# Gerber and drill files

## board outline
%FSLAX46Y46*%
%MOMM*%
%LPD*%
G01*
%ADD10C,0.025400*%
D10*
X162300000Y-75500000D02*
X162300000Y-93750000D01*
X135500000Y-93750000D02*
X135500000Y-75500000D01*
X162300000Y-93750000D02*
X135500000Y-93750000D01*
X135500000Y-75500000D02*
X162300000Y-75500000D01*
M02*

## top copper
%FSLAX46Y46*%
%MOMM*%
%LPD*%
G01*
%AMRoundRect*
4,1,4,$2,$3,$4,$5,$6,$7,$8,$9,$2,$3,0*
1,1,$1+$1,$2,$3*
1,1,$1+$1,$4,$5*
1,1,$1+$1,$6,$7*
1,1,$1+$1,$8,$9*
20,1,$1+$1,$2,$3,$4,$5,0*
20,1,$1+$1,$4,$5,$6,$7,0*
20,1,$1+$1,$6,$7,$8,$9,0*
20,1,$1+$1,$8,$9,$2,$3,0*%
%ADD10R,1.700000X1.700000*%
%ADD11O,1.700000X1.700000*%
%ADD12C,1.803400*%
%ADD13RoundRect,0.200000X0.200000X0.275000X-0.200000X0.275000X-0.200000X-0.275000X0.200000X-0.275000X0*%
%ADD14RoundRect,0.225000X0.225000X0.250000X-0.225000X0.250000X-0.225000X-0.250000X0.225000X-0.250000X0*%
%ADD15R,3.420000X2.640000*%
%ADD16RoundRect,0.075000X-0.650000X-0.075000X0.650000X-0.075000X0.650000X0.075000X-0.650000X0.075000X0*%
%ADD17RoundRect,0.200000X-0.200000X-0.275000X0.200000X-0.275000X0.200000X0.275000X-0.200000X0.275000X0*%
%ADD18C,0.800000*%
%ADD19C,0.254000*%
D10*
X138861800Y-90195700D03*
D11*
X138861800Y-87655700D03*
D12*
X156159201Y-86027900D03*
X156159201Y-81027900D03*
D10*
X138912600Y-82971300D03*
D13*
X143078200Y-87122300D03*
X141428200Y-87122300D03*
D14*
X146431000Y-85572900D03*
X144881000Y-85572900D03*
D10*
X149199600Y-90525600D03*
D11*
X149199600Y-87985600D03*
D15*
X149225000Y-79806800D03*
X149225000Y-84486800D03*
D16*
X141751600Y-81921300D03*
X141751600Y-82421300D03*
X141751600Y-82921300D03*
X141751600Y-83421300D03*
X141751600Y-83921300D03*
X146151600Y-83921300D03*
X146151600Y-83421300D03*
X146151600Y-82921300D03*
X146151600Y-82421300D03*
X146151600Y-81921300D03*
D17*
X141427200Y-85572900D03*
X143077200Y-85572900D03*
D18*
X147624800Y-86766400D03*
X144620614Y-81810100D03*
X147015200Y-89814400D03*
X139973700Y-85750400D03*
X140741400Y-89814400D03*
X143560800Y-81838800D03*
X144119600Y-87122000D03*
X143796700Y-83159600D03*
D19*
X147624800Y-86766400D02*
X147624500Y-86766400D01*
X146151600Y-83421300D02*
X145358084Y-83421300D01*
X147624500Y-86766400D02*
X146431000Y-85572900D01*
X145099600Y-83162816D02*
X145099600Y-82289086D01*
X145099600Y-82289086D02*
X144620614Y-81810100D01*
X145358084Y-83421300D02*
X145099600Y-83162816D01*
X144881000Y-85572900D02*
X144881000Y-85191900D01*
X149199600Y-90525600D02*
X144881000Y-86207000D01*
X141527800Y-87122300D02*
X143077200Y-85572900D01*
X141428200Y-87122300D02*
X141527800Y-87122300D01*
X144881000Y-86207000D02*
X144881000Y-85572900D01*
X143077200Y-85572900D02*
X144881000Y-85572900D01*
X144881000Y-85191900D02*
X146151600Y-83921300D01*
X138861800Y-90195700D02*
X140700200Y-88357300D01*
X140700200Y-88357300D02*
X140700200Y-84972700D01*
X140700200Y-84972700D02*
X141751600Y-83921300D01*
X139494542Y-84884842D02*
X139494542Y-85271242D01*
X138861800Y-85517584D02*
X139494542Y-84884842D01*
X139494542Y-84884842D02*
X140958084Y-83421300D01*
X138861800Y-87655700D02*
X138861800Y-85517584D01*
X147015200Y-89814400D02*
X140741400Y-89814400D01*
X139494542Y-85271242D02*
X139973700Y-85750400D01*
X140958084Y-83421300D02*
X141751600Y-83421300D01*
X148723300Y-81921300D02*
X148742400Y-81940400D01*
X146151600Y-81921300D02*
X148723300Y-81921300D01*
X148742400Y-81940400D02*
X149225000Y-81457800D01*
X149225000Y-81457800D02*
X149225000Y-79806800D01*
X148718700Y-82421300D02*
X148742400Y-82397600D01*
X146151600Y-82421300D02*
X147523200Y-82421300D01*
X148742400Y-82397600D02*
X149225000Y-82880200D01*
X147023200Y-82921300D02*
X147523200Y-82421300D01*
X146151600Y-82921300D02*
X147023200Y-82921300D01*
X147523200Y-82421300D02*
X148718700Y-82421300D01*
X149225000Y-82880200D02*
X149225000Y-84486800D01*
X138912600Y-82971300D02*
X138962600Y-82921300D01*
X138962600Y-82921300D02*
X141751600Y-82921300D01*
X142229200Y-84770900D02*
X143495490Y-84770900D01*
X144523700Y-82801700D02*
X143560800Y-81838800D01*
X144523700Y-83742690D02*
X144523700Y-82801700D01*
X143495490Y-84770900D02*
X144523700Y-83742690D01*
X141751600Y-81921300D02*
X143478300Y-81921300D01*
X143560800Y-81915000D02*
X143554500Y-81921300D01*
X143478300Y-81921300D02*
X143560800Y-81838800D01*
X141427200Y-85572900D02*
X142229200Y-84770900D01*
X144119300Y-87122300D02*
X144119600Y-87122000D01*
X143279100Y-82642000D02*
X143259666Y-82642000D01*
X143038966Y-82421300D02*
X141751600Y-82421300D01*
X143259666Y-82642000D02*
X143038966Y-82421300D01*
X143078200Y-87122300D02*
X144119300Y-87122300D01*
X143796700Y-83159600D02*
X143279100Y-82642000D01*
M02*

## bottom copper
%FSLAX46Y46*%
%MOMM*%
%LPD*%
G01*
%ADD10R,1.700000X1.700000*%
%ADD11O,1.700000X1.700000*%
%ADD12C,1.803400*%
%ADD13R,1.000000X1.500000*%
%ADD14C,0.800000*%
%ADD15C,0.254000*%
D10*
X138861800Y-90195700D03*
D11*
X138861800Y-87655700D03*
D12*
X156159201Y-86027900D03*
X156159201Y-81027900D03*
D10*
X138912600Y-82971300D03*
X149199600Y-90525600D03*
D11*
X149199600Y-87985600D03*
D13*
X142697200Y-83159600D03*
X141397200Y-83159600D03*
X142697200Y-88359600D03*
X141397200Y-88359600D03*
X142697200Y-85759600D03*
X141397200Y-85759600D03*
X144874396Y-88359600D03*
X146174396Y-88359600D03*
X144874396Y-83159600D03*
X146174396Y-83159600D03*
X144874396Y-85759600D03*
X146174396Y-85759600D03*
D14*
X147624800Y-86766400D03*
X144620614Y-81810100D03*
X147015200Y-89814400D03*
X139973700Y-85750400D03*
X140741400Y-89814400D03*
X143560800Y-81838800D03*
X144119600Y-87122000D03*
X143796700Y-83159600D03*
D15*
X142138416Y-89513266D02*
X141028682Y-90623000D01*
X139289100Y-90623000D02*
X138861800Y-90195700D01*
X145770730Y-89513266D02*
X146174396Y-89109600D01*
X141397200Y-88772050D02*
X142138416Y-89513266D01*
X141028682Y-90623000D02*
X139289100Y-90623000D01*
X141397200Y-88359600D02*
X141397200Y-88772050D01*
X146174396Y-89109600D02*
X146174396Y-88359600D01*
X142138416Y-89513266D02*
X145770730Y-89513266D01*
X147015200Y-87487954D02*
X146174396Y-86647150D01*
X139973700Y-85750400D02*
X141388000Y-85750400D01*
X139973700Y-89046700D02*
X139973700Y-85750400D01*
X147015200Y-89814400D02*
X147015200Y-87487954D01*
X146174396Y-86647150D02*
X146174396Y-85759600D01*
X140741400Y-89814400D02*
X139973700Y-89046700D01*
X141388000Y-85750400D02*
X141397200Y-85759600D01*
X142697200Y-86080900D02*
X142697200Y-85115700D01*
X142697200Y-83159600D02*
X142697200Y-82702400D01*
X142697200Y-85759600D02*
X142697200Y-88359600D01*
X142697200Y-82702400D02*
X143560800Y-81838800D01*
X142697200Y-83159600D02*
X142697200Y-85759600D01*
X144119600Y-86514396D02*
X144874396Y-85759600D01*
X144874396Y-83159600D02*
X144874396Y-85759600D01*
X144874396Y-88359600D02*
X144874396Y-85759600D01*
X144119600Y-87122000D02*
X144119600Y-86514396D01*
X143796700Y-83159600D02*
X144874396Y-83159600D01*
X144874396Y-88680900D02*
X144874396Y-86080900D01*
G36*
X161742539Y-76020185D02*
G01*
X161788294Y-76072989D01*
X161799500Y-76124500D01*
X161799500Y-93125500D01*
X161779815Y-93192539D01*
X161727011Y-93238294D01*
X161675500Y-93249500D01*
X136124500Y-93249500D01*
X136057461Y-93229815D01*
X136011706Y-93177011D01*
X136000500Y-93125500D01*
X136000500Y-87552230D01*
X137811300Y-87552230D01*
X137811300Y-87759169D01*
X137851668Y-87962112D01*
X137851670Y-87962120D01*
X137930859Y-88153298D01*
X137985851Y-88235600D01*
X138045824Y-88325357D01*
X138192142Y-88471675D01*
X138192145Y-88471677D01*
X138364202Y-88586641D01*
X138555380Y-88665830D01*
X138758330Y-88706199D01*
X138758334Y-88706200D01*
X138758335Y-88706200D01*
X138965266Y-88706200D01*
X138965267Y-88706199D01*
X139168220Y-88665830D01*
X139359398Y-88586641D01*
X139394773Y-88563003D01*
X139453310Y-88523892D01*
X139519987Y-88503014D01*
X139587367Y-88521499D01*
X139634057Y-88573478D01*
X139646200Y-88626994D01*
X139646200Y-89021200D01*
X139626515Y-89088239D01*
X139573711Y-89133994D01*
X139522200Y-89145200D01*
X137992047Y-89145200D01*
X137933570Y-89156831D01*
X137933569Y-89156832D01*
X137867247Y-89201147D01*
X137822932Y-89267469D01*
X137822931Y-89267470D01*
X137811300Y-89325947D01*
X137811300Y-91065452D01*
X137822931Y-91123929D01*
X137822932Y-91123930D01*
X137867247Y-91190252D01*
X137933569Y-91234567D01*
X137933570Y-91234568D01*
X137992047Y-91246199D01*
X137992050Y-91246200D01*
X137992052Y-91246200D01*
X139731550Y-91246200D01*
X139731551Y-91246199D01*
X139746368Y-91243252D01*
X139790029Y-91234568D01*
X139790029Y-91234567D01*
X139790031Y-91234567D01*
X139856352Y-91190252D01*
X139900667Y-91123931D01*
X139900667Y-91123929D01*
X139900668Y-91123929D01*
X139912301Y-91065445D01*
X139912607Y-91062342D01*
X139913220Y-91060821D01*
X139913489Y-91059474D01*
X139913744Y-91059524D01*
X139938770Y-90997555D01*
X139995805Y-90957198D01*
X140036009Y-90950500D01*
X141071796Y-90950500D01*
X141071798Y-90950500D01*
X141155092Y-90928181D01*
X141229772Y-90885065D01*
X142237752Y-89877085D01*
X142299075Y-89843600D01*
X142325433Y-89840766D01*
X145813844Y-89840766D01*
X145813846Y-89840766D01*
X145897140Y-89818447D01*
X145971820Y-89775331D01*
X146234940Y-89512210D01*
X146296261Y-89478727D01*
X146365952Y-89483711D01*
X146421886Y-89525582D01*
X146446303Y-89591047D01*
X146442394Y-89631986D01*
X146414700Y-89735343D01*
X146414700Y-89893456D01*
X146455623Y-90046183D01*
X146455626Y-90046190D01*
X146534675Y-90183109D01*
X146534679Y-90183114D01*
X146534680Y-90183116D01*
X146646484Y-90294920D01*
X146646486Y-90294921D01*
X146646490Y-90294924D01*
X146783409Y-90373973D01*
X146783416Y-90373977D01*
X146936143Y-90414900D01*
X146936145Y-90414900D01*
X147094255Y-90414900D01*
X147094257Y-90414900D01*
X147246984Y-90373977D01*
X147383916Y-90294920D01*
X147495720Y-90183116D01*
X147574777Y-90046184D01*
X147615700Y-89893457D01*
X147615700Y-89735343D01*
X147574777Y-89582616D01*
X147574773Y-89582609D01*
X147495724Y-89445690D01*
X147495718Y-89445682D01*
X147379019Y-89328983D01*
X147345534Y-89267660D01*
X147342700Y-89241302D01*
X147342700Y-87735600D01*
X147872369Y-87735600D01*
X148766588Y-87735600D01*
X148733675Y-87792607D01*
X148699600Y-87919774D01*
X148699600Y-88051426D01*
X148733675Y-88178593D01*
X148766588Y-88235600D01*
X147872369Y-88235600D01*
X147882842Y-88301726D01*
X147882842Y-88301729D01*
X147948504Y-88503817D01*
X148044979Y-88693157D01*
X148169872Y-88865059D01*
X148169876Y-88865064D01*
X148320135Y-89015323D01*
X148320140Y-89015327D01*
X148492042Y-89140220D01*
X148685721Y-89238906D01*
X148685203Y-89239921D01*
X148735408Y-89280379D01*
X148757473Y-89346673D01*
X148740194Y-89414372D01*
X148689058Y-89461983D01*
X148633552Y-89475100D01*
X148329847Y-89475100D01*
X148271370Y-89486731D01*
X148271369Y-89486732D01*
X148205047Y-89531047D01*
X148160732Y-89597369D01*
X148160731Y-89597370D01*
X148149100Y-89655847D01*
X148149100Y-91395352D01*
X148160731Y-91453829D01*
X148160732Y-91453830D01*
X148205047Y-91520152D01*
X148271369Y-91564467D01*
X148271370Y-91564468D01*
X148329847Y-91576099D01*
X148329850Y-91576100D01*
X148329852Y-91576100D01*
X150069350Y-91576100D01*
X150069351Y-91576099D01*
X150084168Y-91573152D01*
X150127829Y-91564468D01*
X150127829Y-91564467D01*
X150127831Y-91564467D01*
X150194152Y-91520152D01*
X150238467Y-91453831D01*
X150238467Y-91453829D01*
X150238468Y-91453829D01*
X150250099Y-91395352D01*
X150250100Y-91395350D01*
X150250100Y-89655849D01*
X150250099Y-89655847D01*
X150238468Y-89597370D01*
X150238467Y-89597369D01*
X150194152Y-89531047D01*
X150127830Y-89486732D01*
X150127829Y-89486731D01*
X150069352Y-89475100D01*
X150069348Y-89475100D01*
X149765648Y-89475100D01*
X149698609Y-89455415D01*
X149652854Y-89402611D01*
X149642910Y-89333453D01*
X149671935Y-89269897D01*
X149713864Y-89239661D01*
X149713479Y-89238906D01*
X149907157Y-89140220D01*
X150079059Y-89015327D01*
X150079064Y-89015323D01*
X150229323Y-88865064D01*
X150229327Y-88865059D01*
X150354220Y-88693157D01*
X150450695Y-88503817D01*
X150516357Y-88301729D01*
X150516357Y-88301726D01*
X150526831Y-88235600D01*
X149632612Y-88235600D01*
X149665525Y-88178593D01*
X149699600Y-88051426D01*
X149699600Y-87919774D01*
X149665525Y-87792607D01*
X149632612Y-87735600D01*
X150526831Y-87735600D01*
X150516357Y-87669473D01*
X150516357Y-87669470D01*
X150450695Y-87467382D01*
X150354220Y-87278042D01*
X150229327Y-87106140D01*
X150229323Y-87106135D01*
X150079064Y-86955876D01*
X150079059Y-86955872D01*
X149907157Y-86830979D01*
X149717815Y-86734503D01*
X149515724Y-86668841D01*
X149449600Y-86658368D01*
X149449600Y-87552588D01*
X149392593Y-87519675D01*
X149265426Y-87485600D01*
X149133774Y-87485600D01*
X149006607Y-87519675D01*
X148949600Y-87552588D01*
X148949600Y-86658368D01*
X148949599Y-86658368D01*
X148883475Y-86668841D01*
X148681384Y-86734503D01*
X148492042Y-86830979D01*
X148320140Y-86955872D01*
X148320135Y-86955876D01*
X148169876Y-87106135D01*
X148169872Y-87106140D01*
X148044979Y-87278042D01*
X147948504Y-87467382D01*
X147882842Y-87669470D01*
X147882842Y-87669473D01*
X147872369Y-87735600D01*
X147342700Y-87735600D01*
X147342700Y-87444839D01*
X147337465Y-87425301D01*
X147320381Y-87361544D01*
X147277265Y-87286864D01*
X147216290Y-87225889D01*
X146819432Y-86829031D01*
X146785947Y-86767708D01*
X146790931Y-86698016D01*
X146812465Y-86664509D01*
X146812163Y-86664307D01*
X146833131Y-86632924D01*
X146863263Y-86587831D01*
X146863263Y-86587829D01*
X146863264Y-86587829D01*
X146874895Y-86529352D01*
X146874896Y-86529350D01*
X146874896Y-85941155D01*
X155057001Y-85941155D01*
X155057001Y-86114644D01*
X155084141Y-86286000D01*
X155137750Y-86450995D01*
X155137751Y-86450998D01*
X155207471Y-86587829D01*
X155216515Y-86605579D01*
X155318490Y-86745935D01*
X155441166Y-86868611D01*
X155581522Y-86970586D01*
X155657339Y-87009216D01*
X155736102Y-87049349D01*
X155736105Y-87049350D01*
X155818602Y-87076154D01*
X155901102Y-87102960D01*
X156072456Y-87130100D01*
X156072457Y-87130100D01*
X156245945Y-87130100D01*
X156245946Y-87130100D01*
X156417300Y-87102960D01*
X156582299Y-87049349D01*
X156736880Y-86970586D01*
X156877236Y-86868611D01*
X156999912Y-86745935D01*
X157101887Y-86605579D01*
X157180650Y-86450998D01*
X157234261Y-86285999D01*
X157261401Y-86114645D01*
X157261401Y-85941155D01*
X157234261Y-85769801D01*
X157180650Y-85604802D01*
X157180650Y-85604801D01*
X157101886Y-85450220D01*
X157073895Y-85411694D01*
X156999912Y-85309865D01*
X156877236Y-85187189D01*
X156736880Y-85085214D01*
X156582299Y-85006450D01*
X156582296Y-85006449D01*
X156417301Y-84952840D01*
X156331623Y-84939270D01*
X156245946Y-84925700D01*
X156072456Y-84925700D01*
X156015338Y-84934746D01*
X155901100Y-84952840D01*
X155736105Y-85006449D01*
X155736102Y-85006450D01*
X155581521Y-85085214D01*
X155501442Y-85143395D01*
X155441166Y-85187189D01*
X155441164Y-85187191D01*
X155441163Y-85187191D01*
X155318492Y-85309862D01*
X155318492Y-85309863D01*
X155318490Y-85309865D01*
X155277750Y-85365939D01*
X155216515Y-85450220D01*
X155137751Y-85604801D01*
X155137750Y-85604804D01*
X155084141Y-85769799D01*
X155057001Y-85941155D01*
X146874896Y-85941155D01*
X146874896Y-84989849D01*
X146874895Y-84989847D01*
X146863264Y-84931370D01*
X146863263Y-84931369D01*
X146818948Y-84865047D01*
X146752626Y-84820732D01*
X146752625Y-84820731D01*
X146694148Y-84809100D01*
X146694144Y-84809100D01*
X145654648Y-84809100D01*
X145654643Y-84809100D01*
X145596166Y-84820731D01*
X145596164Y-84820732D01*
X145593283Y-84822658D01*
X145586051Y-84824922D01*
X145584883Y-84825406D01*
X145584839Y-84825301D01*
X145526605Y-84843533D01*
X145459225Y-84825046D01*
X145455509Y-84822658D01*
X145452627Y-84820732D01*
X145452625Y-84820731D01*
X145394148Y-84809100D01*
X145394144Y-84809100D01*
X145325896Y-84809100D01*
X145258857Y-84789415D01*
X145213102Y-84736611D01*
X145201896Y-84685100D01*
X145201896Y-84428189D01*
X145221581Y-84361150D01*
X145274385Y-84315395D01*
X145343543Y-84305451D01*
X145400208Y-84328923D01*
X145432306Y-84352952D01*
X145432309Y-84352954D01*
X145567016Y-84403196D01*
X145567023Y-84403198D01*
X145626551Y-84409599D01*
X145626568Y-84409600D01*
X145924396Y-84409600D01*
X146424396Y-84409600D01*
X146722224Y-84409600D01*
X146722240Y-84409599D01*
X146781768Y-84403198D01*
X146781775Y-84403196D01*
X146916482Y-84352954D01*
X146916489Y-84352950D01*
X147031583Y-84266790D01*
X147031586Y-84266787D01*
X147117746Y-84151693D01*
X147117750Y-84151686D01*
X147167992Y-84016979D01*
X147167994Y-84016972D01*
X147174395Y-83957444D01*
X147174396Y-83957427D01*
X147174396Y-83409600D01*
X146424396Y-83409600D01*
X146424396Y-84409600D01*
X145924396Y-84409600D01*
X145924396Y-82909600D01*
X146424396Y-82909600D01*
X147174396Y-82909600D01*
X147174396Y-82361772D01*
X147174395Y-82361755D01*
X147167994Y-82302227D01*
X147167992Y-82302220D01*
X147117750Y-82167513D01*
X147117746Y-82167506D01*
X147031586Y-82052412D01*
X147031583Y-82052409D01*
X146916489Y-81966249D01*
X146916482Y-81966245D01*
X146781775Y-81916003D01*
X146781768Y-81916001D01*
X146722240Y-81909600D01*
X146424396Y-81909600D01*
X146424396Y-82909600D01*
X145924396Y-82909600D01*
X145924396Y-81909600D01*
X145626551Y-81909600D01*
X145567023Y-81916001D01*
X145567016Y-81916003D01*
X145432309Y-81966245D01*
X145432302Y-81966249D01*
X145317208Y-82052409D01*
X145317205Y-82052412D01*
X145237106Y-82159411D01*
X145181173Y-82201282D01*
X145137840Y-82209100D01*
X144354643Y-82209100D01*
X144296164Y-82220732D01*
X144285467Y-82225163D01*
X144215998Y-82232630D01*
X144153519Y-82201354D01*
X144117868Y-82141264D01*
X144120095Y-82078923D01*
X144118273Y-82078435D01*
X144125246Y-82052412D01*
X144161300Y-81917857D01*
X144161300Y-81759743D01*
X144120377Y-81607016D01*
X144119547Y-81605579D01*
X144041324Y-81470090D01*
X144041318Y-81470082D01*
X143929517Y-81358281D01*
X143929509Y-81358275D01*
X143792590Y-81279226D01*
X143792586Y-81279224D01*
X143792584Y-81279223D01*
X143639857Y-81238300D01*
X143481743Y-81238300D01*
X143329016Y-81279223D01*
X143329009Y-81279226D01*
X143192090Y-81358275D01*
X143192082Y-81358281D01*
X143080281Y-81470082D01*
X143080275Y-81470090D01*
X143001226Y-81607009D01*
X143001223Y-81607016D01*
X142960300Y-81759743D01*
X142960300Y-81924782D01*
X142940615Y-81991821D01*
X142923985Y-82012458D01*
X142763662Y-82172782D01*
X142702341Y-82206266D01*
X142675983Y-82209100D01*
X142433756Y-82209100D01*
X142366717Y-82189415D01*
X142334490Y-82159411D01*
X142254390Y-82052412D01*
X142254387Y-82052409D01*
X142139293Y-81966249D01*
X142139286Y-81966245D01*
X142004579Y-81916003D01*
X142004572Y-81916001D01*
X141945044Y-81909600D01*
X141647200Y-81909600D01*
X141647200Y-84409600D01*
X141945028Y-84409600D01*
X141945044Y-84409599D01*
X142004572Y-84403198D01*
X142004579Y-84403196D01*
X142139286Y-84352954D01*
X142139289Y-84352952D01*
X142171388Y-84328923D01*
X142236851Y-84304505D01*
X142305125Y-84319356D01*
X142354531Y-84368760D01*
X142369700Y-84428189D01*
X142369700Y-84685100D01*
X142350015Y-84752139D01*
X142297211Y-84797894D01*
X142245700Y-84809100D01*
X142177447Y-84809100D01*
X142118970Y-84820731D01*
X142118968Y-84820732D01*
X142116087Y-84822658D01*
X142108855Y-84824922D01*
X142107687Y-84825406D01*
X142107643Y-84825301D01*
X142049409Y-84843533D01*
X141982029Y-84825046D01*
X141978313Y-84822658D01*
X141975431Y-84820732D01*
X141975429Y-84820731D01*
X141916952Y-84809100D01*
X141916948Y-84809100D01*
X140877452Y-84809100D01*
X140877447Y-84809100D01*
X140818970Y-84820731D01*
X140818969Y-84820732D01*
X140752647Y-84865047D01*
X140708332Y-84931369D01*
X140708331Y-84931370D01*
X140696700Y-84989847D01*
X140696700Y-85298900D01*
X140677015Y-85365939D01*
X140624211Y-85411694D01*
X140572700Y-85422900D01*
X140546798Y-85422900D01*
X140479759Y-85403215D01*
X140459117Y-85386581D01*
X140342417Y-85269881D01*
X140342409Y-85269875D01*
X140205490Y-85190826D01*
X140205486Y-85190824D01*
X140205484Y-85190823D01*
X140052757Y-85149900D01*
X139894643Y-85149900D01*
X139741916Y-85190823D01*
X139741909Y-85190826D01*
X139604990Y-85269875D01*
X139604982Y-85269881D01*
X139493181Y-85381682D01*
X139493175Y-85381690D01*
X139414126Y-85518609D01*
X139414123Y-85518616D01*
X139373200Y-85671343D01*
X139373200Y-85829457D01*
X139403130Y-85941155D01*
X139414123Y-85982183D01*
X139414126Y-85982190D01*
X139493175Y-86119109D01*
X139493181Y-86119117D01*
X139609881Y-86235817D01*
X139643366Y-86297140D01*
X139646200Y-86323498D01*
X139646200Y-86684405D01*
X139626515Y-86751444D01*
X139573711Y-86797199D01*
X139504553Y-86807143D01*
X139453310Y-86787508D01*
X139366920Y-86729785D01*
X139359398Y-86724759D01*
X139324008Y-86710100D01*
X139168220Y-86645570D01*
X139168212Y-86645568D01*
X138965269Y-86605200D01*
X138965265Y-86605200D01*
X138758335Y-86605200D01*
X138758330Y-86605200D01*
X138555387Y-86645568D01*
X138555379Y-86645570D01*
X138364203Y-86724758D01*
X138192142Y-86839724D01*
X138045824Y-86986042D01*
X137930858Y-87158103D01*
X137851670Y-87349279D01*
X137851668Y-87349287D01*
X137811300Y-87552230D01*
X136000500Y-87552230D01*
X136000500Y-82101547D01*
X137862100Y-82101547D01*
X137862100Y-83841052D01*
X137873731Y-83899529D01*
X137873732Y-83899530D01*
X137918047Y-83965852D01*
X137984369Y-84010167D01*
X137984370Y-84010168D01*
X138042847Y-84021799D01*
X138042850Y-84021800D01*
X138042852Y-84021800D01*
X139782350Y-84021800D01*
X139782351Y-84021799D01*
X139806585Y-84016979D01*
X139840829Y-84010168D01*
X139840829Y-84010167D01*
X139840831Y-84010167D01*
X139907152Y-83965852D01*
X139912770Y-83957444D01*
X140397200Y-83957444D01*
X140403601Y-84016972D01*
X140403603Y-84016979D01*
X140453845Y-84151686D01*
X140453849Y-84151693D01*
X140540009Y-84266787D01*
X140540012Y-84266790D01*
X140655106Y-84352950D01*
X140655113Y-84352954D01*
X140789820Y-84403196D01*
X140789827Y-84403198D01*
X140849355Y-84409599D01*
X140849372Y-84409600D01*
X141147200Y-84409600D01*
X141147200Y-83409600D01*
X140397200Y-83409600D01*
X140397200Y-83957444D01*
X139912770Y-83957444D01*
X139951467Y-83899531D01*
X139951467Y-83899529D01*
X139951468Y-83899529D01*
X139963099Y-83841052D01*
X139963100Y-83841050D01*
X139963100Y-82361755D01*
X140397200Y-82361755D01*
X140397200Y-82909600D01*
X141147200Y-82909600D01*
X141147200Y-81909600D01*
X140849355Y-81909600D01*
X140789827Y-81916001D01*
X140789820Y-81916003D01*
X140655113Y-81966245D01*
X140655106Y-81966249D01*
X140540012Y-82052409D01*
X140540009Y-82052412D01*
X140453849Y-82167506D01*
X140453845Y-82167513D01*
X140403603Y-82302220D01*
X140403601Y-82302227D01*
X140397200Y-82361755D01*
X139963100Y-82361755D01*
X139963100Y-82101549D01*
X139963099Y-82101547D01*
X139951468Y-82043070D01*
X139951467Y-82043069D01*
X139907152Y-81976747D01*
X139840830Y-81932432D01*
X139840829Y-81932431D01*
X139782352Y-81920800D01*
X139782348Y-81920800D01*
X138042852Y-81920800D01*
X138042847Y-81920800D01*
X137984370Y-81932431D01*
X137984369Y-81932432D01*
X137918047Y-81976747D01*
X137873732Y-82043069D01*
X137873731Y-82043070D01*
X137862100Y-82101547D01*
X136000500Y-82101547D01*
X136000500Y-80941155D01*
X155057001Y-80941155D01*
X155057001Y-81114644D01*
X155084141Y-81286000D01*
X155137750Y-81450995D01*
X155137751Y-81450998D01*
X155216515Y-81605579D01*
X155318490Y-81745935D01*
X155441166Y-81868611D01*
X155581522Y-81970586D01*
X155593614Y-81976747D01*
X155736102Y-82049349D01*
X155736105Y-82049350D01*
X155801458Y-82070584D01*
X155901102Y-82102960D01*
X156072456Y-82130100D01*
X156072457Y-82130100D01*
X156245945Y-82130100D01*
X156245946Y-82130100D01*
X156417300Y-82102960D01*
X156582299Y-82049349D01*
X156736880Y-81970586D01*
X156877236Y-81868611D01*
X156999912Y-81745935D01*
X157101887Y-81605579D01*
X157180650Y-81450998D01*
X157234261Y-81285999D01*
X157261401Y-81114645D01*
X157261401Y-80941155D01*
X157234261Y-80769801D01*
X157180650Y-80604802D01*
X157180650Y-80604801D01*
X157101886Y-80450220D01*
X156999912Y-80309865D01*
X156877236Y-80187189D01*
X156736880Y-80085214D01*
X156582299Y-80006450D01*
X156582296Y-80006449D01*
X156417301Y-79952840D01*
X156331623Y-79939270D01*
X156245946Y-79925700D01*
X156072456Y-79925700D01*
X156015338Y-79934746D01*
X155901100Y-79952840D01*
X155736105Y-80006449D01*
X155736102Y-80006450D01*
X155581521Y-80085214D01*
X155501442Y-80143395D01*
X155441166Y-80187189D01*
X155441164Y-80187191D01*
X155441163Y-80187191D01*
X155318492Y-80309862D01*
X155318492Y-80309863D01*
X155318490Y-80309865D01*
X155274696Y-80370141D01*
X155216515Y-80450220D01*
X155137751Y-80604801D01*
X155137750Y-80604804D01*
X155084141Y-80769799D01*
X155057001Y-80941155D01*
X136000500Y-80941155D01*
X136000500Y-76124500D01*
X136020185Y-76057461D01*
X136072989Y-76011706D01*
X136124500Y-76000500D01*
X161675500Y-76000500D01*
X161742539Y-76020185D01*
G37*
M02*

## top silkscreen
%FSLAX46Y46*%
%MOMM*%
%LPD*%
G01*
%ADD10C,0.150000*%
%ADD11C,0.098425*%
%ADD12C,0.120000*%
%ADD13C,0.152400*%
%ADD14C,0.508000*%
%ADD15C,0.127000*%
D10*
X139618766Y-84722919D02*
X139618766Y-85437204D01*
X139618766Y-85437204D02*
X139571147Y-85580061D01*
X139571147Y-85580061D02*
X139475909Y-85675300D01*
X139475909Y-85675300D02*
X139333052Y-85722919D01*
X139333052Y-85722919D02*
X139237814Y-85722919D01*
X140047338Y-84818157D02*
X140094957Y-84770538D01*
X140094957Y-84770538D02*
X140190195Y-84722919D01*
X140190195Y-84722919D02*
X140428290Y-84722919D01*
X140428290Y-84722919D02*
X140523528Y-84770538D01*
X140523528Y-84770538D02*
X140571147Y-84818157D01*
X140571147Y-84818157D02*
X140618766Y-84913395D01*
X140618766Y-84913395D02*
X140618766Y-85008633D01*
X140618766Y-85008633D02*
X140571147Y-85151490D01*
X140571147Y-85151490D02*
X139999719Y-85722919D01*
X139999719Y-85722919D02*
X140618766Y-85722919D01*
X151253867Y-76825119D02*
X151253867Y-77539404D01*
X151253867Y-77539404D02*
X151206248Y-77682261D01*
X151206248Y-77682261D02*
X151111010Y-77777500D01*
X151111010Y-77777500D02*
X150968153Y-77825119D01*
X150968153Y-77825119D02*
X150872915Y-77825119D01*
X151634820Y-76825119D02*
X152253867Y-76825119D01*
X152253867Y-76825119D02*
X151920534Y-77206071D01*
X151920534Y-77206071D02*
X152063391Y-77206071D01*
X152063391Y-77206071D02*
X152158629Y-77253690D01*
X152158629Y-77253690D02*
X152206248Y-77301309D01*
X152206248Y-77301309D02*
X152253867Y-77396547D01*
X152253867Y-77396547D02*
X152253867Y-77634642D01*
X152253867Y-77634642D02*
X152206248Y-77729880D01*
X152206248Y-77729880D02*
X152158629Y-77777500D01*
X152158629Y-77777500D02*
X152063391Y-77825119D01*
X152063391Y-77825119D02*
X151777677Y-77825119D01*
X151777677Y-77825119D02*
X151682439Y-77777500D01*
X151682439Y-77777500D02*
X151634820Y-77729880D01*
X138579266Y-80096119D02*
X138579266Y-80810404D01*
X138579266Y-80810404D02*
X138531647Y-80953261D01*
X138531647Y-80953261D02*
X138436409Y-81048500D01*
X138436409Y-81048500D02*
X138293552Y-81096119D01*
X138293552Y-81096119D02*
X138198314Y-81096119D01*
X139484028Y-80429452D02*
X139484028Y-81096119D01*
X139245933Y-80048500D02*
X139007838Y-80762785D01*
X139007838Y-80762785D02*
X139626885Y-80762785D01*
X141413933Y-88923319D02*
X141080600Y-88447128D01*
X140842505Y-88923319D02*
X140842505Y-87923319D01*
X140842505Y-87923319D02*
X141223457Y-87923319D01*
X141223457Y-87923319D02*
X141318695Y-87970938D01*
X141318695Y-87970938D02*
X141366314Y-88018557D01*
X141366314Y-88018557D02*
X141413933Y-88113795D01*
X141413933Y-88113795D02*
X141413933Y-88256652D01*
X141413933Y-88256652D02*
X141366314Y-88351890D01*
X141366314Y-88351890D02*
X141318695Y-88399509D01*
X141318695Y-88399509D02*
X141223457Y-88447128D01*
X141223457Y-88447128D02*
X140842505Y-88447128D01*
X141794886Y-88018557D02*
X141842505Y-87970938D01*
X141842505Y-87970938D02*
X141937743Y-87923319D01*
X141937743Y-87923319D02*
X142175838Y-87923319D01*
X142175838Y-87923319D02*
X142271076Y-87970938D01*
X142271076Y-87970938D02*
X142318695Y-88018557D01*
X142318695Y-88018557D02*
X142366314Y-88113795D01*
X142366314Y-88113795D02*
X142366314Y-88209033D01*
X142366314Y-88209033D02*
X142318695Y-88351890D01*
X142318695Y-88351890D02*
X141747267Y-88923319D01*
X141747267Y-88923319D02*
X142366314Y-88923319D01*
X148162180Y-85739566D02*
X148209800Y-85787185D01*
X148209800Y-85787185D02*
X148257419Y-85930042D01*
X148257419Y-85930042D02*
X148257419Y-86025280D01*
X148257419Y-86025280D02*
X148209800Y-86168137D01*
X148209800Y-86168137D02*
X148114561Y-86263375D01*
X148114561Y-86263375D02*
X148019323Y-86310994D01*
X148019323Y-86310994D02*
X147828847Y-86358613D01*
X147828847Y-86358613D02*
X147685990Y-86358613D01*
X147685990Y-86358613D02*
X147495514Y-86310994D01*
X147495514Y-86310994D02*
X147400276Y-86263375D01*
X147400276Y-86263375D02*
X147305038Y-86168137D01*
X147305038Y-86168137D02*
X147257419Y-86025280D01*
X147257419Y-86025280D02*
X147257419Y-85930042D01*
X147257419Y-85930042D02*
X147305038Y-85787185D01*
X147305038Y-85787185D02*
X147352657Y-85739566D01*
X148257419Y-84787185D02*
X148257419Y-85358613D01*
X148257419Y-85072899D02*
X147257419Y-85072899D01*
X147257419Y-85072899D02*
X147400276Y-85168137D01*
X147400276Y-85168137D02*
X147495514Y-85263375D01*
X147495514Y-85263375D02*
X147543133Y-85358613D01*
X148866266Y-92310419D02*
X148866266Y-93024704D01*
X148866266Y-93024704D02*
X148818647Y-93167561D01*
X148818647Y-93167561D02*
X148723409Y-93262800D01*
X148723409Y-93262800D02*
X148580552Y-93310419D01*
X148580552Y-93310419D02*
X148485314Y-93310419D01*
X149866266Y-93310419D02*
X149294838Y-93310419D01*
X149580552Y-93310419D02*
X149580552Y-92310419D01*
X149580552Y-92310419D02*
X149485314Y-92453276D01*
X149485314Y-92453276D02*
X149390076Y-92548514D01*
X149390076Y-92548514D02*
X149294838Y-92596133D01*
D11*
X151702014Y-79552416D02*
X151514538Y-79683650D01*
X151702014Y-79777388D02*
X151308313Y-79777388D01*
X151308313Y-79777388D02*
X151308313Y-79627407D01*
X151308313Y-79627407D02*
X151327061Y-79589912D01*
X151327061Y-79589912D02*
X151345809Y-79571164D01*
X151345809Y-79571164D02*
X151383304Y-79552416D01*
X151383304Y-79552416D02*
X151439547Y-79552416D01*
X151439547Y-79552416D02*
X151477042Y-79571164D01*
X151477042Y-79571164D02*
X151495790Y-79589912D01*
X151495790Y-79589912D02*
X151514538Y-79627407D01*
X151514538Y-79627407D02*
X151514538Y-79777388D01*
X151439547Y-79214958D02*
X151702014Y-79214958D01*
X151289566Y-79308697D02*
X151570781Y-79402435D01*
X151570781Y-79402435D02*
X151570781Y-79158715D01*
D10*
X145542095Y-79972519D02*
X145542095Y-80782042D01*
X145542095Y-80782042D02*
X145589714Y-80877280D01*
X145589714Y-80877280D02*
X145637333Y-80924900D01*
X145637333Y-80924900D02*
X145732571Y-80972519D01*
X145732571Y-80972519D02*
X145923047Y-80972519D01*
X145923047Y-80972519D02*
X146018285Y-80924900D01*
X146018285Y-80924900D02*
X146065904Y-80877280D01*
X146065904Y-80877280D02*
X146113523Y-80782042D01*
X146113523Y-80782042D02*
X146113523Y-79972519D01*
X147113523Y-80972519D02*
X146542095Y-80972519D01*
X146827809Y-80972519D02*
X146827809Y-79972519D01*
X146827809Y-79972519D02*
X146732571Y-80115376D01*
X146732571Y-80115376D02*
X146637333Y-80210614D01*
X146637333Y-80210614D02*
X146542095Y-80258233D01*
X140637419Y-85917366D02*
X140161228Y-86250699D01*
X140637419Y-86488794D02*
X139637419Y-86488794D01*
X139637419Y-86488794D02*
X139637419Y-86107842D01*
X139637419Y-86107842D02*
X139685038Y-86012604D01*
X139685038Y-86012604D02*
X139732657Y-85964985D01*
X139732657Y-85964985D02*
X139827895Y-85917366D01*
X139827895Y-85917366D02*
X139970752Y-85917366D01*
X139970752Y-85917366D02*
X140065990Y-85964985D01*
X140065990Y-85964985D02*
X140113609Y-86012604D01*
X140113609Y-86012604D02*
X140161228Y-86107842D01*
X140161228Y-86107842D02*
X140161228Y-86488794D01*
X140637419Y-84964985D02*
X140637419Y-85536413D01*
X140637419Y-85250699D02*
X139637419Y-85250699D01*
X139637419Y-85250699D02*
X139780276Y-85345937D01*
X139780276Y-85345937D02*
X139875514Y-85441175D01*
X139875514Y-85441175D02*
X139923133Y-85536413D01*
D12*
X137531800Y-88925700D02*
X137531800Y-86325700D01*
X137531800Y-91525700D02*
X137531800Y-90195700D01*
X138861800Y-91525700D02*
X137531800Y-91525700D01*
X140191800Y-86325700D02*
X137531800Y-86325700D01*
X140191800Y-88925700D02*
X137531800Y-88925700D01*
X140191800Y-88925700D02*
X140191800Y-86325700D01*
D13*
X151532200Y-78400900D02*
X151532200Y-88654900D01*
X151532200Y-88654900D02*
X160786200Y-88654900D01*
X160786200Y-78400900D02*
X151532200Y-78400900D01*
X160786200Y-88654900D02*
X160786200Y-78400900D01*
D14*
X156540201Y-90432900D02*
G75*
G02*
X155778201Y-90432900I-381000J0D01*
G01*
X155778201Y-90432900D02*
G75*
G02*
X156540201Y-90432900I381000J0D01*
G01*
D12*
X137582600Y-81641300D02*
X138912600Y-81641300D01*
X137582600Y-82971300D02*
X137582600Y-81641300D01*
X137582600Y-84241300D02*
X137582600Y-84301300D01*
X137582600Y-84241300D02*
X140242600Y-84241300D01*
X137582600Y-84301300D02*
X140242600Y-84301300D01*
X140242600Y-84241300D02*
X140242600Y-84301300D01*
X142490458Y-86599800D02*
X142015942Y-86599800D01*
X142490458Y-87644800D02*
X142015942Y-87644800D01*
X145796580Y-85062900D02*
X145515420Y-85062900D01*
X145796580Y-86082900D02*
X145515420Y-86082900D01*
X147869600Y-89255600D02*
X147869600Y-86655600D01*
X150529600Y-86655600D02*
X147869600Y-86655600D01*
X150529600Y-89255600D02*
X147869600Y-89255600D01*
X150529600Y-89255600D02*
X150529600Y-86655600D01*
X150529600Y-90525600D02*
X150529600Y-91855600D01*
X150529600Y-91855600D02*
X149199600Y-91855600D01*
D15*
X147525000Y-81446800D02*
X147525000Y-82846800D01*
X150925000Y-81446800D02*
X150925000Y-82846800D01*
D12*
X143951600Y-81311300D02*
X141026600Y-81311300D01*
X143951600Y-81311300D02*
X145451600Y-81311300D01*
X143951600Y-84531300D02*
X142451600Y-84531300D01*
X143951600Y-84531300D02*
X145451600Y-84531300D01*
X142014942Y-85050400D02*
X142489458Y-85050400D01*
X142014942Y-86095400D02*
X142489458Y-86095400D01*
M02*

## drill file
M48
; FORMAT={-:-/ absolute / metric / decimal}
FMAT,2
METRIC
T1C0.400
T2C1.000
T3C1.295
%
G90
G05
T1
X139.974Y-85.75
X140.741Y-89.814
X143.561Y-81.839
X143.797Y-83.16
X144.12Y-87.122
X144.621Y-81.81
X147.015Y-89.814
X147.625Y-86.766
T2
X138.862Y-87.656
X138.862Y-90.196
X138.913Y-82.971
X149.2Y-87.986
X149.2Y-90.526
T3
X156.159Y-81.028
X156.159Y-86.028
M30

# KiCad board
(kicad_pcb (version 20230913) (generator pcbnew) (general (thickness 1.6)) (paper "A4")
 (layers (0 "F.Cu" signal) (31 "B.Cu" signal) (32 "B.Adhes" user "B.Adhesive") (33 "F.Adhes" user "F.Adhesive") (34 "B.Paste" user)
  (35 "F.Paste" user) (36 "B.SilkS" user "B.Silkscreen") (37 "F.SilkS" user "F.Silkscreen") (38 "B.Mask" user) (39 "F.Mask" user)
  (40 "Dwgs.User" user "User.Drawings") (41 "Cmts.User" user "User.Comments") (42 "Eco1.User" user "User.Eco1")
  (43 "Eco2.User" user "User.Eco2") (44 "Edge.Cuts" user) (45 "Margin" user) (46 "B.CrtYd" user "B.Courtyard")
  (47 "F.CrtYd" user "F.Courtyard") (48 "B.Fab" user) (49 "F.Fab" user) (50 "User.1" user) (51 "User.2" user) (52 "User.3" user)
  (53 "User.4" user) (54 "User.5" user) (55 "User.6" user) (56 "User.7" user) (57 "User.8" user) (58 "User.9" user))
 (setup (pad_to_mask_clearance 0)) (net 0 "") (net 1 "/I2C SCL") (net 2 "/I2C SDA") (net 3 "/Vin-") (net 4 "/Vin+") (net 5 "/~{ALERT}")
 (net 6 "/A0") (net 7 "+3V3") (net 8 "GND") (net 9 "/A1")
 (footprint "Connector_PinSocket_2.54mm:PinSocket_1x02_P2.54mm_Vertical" (layer "F.Cu") (at 138.8618 90.1957 180)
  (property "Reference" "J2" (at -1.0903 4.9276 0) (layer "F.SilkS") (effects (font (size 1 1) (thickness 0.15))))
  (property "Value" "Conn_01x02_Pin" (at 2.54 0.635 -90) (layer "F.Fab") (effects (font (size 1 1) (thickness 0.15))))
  (fp_line (start 1.33 1.27) (end 1.33 3.87) (stroke (width 0.12) (type solid)) (layer "F.SilkS"))
  (fp_line (start 1.33 -1.33) (end 1.33 0) (stroke (width 0.12) (type solid)) (layer "F.SilkS"))
  (fp_line (start 0 -1.33) (end 1.33 -1.33) (stroke (width 0.12) (type solid)) (layer "F.SilkS"))
  (fp_line (start -1.33 3.87) (end 1.33 3.87) (stroke (width 0.12) (type solid)) (layer "F.SilkS"))
  (fp_line (start -1.33 1.27) (end 1.33 1.27) (stroke (width 0.12) (type solid)) (layer "F.SilkS"))
  (fp_line (start -1.33 1.27) (end -1.33 3.87) (stroke (width 0.12) (type solid)) (layer "F.SilkS"))
  (pad "1" thru_hole rect (at 0 0 180) (size 1.7 1.7) (drill 1) (layers "*.Cu" "*.Mask") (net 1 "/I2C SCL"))
  (pad "2" thru_hole oval (at 0 2.54 180) (size 1.7 1.7) (drill 1) (layers "*.Cu" "*.Mask") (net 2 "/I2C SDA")))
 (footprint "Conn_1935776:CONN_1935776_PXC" (layer "F.Cu") (at 156.159201 86.0279 90)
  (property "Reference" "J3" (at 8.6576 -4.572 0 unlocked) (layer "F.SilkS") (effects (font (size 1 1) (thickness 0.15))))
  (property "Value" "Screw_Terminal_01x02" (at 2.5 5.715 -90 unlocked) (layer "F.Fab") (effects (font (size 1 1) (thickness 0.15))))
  (fp_line (start 7.627 -4.627001) (end -2.627 -4.627001) (stroke (width 0.1524) (type solid)) (layer "F.SilkS"))
  (fp_line (start -2.627 -4.627001) (end -2.627 4.626999) (stroke (width 0.1524) (type solid)) (layer "F.SilkS"))
  (fp_line (start 7.627 4.626999) (end 7.627 -4.627001) (stroke (width 0.1524) (type solid)) (layer "F.SilkS"))
  (fp_line (start -2.627 4.626999) (end 7.627 4.626999) (stroke (width 0.1524) (type solid)) (layer "F.SilkS"))
  (fp_circle (center -4.405 0) (end -4.024 0) (stroke (width 0.508) (type solid)) (fill none) (layer "F.SilkS"))
  (pad "1" thru_hole circle (at 0 0 90) (size 1.8034 1.8034) (drill 1.2954) (layers "*.Cu" "*.Mask") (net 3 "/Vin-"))
  (pad "2" thru_hole circle (at 5 0 90) (size 1.8034 1.8034) (drill 1.2954) (layers "*.Cu" "*.Mask") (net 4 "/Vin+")))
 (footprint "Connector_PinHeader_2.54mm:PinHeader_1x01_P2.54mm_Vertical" (layer "F.Cu") (at 138.9126 82.9713)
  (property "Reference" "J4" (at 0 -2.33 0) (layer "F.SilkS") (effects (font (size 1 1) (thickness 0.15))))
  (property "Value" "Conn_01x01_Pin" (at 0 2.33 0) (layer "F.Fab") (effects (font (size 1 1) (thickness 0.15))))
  (fp_line (start -1.33 -1.33) (end 0 -1.33) (stroke (width 0.12) (type solid)) (layer "F.SilkS"))
  (fp_line (start -1.33 0) (end -1.33 -1.33) (stroke (width 0.12) (type solid)) (layer "F.SilkS"))
  (fp_line (start -1.33 1.27) (end -1.33 1.33) (stroke (width 0.12) (type solid)) (layer "F.SilkS"))
  (fp_line (start -1.33 1.27) (end 1.33 1.27) (stroke (width 0.12) (type solid)) (layer "F.SilkS"))
  (fp_line (start -1.33 1.33) (end 1.33 1.33) (stroke (width 0.12) (type solid)) (layer "F.SilkS"))
  (fp_line (start 1.33 1.27) (end 1.33 1.33) (stroke (width 0.12) (type solid)) (layer "F.SilkS"))
  (pad "1" thru_hole rect (at 0 0) (size 1.7 1.7) (drill 1) (layers "*.Cu" "*.Mask") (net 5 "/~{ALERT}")))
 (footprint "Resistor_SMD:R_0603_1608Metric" (layer "F.Cu") (at 142.2532 87.1223 180)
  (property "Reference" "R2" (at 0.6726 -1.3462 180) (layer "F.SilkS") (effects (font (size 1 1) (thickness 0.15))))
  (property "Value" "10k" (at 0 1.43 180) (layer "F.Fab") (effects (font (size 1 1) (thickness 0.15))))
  (fp_line (start -0.237258 0.5225) (end 0.237258 0.5225) (stroke (width 0.12) (type solid)) (layer "F.SilkS"))
  (fp_line (start -0.237258 -0.5225) (end 0.237258 -0.5225) (stroke (width 0.12) (type solid)) (layer "F.SilkS"))
  (pad "1" smd roundrect (at -0.825 0 180) (size 0.8 0.95) (layers "F.Cu" "F.Paste" "F.Mask") (roundrect_rratio 0.25) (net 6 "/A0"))
  (pad "2" smd roundrect (at 0.825 0 180) (size 0.8 0.95) (layers "F.Cu" "F.Paste" "F.Mask") (roundrect_rratio 0.25) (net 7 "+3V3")))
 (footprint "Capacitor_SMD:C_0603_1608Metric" (layer "F.Cu") (at 145.656 85.5729 180)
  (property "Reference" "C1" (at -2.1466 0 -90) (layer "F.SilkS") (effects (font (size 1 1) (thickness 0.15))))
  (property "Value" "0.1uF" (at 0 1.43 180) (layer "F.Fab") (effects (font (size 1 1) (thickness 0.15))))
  (fp_line (start -0.14058 0.51) (end 0.14058 0.51) (stroke (width 0.12) (type solid)) (layer "F.SilkS"))
  (fp_line (start -0.14058 -0.51) (end 0.14058 -0.51) (stroke (width 0.12) (type solid)) (layer "F.SilkS"))
  (pad "1" smd roundrect (at -0.775 0 180) (size 0.9 0.95) (layers "F.Cu" "F.Paste" "F.Mask") (roundrect_rratio 0.25) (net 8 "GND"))
  (pad "2" smd roundrect (at 0.775 0 180) (size 0.9 0.95) (layers "F.Cu" "F.Paste" "F.Mask") (roundrect_rratio 0.25) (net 7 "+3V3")))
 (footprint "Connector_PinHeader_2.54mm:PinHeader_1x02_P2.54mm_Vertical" (layer "F.Cu") (at 149.1996 90.5256 180)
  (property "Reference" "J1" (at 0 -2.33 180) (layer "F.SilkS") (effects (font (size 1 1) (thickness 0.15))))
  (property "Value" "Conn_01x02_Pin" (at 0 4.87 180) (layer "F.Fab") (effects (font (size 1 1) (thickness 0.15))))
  (fp_line (start 1.33 1.27) (end 1.33 3.87) (stroke (width 0.12) (type solid)) (layer "F.SilkS"))
  (fp_line (start -1.33 3.87) (end 1.33 3.87) (stroke (width 0.12) (type solid)) (layer "F.SilkS"))
  (fp_line (start -1.33 1.27) (end 1.33 1.27) (stroke (width 0.12) (type solid)) (layer "F.SilkS"))
  (fp_line (start -1.33 1.27) (end -1.33 3.87) (stroke (width 0.12) (type solid)) (layer "F.SilkS"))
  (fp_line (start -1.33 0) (end -1.33 -1.33) (stroke (width 0.12) (type solid)) (layer "F.SilkS"))
  (fp_line (start -1.33 -1.33) (end 0 -1.33) (stroke (width 0.12) (type solid)) (layer "F.SilkS"))
  (pad "1" thru_hole rect (at 0 0 180) (size 1.7 1.7) (drill 1) (layers "*.Cu" "*.Mask") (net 7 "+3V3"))
  (pad "2" thru_hole oval (at 0 2.54 180) (size 1.7 1.7) (drill 1) (layers "*.Cu" "*.Mask") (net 8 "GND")))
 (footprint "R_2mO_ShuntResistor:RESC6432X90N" (layer "F.Cu") (at 149.225 82.1468 -90)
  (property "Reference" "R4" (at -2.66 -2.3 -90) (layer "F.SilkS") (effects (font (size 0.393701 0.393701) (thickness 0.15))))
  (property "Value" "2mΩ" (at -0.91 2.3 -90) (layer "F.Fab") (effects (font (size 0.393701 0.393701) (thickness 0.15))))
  (fp_line (start -0.7 1.7) (end 0.7 1.7) (stroke (width 0.127) (type solid)) (layer "F.SilkS"))
  (fp_line (start -0.7 -1.7) (end 0.7 -1.7) (stroke (width 0.127) (type solid)) (layer "F.SilkS"))
  (pad "1" smd rect (at -2.34 0 270) (size 2.64 3.42) (layers "F.Cu" "F.Paste" "F.Mask") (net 4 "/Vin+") (solder_mask_margin 0.102))
  (pad "2" smd rect (at 2.34 0 270) (size 2.64 3.42) (layers "F.Cu" "F.Paste" "F.Mask") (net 3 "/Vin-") (solder_mask_margin 0.102)))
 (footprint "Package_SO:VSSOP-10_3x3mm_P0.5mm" (layer "F.Cu") (at 143.9516 82.9213)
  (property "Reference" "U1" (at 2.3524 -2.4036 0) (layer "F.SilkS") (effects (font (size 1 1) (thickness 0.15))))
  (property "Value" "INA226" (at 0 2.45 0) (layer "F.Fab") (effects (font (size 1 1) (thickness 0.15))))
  (fp_line (start 0 -1.61) (end -2.925 -1.61) (stroke (width 0.12) (type solid)) (layer "F.SilkS"))
  (fp_line (start 0 -1.61) (end 1.5 -1.61) (stroke (width 0.12) (type solid)) (layer "F.SilkS"))
  (fp_line (start 0 1.61) (end -1.5 1.61) (stroke (width 0.12) (type solid)) (layer "F.SilkS"))
  (fp_line (start 0 1.61) (end 1.5 1.61) (stroke (width 0.12) (type solid)) (layer "F.SilkS"))
  (pad "1" smd roundrect (at -2.2 -1) (size 1.45 0.3) (layers "F.Cu" "F.Paste" "F.Mask") (roundrect_rratio 0.25) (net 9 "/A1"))
  (pad "2" smd roundrect (at -2.2 -0.5) (size 1.45 0.3) (layers "F.Cu" "F.Paste" "F.Mask") (roundrect_rratio 0.25) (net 6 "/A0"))
  (pad "3" smd roundrect (at -2.2 0) (size 1.45 0.3) (layers "F.Cu" "F.Paste" "F.Mask") (roundrect_rratio 0.25) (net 5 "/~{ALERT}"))
  (pad "4" smd roundrect (at -2.2 0.5) (size 1.45 0.3) (layers "F.Cu" "F.Paste" "F.Mask") (roundrect_rratio 0.25) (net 2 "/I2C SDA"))
  (pad "5" smd roundrect (at -2.2 1) (size 1.45 0.3) (layers "F.Cu" "F.Paste" "F.Mask") (roundrect_rratio 0.25) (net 1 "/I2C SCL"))
  (pad "6" smd roundrect (at 2.2 1) (size 1.45 0.3) (layers "F.Cu" "F.Paste" "F.Mask") (roundrect_rratio 0.25) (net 7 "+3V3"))
  (pad "7" smd roundrect (at 2.2 0.5) (size 1.45 0.3) (layers "F.Cu" "F.Paste" "F.Mask") (roundrect_rratio 0.25) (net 8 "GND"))
  (pad "8" smd roundrect (at 2.2 0) (size 1.45 0.3) (layers "F.Cu" "F.Paste" "F.Mask") (roundrect_rratio 0.25) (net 3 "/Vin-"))
  (pad "9" smd roundrect (at 2.2 -0.5) (size 1.45 0.3) (layers "F.Cu" "F.Paste" "F.Mask") (roundrect_rratio 0.25) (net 3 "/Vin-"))
  (pad "10" smd roundrect (at 2.2 -1) (size 1.45 0.3) (layers "F.Cu" "F.Paste" "F.Mask") (roundrect_rratio 0.25) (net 4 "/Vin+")))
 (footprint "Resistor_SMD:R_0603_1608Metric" (layer "F.Cu") (at 142.2522 85.5729)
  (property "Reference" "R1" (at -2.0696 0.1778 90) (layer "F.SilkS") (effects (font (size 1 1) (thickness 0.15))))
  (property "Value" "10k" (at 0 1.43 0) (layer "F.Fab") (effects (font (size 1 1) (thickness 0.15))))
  (fp_line (start -0.237258 -0.5225) (end 0.237258 -0.5225) (stroke (width 0.12) (type solid)) (layer "F.SilkS"))
  (fp_line (start -0.237258 0.5225) (end 0.237258 0.5225) (stroke (width 0.12) (type solid)) (layer "F.SilkS"))
  (pad "1" smd roundrect (at -0.825 0) (size 0.8 0.95) (layers "F.Cu" "F.Paste" "F.Mask") (roundrect_rratio 0.25) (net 9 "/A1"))
  (pad "2" smd roundrect (at 0.825 0) (size 0.8 0.95) (layers "F.Cu" "F.Paste" "F.Mask") (roundrect_rratio 0.25) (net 7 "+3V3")))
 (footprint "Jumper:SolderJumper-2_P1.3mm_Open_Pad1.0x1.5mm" (layer "B.Cu") (at 142.0472 83.1596 180)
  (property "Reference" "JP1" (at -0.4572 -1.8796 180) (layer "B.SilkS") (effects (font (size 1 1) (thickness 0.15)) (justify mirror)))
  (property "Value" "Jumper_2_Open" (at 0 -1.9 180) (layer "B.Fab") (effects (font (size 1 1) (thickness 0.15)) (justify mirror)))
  (pad "1" smd rect (at -0.65 0 180) (size 1 1.5) (layers "B.Cu" "B.Mask") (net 9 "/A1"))
  (pad "2" smd rect (at 0.65 0 180) (size 1 1.5) (layers "B.Cu" "B.Mask") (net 8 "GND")))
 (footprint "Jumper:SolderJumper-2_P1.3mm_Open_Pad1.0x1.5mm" (layer "B.Cu") (at 142.0472 88.3596 180)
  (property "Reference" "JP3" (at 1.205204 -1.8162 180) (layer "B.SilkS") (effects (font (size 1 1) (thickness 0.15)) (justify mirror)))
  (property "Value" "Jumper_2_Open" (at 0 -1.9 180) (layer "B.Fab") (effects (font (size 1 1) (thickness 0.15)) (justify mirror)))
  (pad "1" smd rect (at -0.65 0 180) (size 1 1.5) (layers "B.Cu" "B.Mask") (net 9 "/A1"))
  (pad "2" smd rect (at 0.65 0 180) (size 1 1.5) (layers "B.Cu" "B.Mask") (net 1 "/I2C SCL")))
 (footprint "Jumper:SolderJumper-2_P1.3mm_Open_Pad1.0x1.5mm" (layer "B.Cu") (at 142.0472 85.7596 180)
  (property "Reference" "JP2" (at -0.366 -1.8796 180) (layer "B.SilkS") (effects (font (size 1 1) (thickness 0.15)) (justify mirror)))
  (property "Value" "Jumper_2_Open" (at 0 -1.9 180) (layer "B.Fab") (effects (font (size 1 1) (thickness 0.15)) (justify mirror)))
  (pad "1" smd rect (at -0.65 0 180) (size 1 1.5) (layers "B.Cu" "B.Mask") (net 9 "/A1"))
  (pad "2" smd rect (at 0.65 0 180) (size 1 1.5) (layers "B.Cu" "B.Mask") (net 2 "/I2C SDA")))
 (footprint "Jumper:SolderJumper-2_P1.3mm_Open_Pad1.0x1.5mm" (layer "B.Cu") (at 145.524396 88.3596)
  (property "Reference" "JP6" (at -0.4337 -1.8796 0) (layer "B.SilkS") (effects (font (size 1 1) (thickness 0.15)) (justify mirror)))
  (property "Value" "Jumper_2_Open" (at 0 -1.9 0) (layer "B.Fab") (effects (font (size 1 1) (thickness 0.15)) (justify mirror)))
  (pad "1" smd rect (at -0.65 0) (size 1 1.5) (layers "B.Cu" "B.Mask") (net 6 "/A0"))
  (pad "2" smd rect (at 0.65 0) (size 1 1.5) (layers "B.Cu" "B.Mask") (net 1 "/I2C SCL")))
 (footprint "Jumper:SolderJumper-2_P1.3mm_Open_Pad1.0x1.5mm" (layer "B.Cu") (at 145.524396 83.1596)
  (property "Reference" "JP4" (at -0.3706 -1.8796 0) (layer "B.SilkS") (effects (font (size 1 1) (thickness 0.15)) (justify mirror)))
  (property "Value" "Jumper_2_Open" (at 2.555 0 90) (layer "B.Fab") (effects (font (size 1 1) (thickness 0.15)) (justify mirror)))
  (pad "1" smd rect (at -0.65 0) (size 1 1.5) (layers "B.Cu" "B.Mask") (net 6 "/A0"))
  (pad "2" smd rect (at 0.65 0) (size 1 1.5) (layers "B.Cu" "B.Mask") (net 8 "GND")))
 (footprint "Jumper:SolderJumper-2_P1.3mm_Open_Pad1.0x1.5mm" (layer "B.Cu") (at 145.524396 85.7596)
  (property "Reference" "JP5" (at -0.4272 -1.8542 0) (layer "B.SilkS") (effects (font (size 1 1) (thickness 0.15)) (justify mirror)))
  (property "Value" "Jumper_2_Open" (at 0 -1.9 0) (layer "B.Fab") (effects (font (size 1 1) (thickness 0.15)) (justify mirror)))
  (pad "1" smd rect (at -0.65 0) (size 1 1.5) (layers "B.Cu" "B.Mask") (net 6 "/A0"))
  (pad "2" smd rect (at 0.65 0) (size 1 1.5) (layers "B.Cu" "B.Mask") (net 2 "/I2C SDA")))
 (gr_line (start 162.3 75.5) (end 162.3 93.75) (stroke (width 0.0254) (type default)) (layer "Edge.Cuts"))
 (gr_line (start 135.5 93.75) (end 135.5 75.5) (stroke (width 0.0254) (type default)) (layer "Edge.Cuts"))
 (gr_line (start 162.3 93.75) (end 135.5 93.75) (stroke (width 0.0254) (type default)) (layer "Edge.Cuts"))
 (gr_line (start 135.5 75.5) (end 162.3 75.5) (stroke (width 0.0254) (type default)) (layer "Edge.Cuts"))
 (segment (start 147.6248 86.7664) (end 147.6245 86.7664) (width 0.254) (layer "F.Cu") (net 8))
 (segment (start 146.1516 83.4213) (end 145.358084 83.4213) (width 0.254) (layer "F.Cu") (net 8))
 (segment (start 147.6245 86.7664) (end 146.431 85.5729) (width 0.254) (layer "F.Cu") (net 8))
 (segment (start 145.0996 83.162816) (end 145.0996 82.289086) (width 0.254) (layer "F.Cu") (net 8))
 (segment (start 145.0996 82.289086) (end 144.620614 81.8101) (width 0.254) (layer "F.Cu") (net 8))
 (segment (start 145.358084 83.4213) (end 145.0996 83.162816) (width 0.254) (layer "F.Cu") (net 8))
 (via (at 147.6248 86.7664) (size 0.8) (drill 0.4) (layers "F.Cu" "B.Cu") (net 8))
 (via (at 144.620614 81.8101) (size 0.8) (drill 0.4) (layers "F.Cu" "B.Cu") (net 8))
 (segment (start 144.881 85.5729) (end 144.881 85.1919) (width 0.254) (layer "F.Cu") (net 7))
 (segment (start 149.1996 90.5256) (end 144.881 86.207) (width 0.254) (layer "F.Cu") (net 7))
 (segment (start 141.5278 87.1223) (end 143.0772 85.5729) (width 0.254) (layer "F.Cu") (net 7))
 (segment (start 141.4282 87.1223) (end 141.5278 87.1223) (width 0.254) (layer "F.Cu") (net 7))
 (segment (start 144.881 86.207) (end 144.881 85.5729) (width 0.254) (layer "F.Cu") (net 7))
 (segment (start 143.0772 85.5729) (end 144.881 85.5729) (width 0.254) (layer "F.Cu") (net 7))
 (segment (start 144.881 85.1919) (end 146.1516 83.9213) (width 0.254) (layer "F.Cu") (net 7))
 (segment (start 138.8618 90.1957) (end 140.7002 88.3573) (width 0.254) (layer "F.Cu") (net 1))
 (segment (start 140.7002 88.3573) (end 140.7002 84.9727) (width 0.254) (layer "F.Cu") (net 1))
 (segment (start 140.7002 84.9727) (end 141.7516 83.9213) (width 0.254) (layer "F.Cu") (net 1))
 (segment (start 142.138416 89.513266) (end 141.028682 90.623) (width 0.254) (layer "B.Cu") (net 1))
 (segment (start 139.2891 90.623) (end 138.8618 90.1957) (width 0.254) (layer "B.Cu") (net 1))
 (segment (start 145.77073 89.513266) (end 146.174396 89.1096) (width 0.254) (layer "B.Cu") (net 1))
 (segment (start 141.3972 88.77205) (end 142.138416 89.513266) (width 0.254) (layer "B.Cu") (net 1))
 (segment (start 141.028682 90.623) (end 139.2891 90.623) (width 0.254) (layer "B.Cu") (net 1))
 (segment (start 141.3972 88.3596) (end 141.3972 88.77205) (width 0.254) (layer "B.Cu") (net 1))
 (segment (start 146.174396 89.1096) (end 146.174396 88.3596) (width 0.254) (layer "B.Cu") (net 1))
 (segment (start 142.138416 89.513266) (end 145.77073 89.513266) (width 0.254) (layer "B.Cu") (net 1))
 (segment (start 139.494542 84.884842) (end 139.494542 85.271242) (width 0.254) (layer "F.Cu") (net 2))
 (segment (start 138.8618 85.517584) (end 139.494542 84.884842) (width 0.254) (layer "F.Cu") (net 2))
 (segment (start 139.494542 84.884842) (end 140.958084 83.4213) (width 0.254) (layer "F.Cu") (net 2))
 (segment (start 138.8618 87.6557) (end 138.8618 85.517584) (width 0.254) (layer "F.Cu") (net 2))
 (segment (start 147.0152 89.8144) (end 140.7414 89.8144) (width 0.254) (layer "F.Cu") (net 2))
 (segment (start 139.494542 85.271242) (end 139.9737 85.7504) (width 0.254) (layer "F.Cu") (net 2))
 (segment (start 140.958084 83.4213) (end 141.7516 83.4213) (width 0.254) (layer "F.Cu") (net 2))
 (via (at 147.0152 89.8144) (size 0.8) (drill 0.4) (layers "F.Cu" "B.Cu") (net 2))
 (via (at 139.9737 85.7504) (size 0.8) (drill 0.4) (layers "F.Cu" "B.Cu") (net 2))
 (via (at 140.7414 89.8144) (size 0.8) (drill 0.4) (layers "F.Cu" "B.Cu") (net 2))
 (segment (start 147.0152 87.487954) (end 146.174396 86.64715) (width 0.254) (layer "B.Cu") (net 2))
 (segment (start 139.9737 85.7504) (end 141.388 85.7504) (width 0.254) (layer "B.Cu") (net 2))
 (segment (start 139.9737 89.0467) (end 139.9737 85.7504) (width 0.254) (layer "B.Cu") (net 2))
 (segment (start 147.0152 89.8144) (end 147.0152 87.487954) (width 0.254) (layer "B.Cu") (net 2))
 (segment (start 146.174396 86.64715) (end 146.174396 85.7596) (width 0.254) (layer "B.Cu") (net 2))
 (segment (start 140.7414 89.8144) (end 139.9737 89.0467) (width 0.254) (layer "B.Cu") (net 2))
 (segment (start 141.388 85.7504) (end 141.3972 85.7596) (width 0.254) (layer "B.Cu") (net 2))
 (segment (start 148.7233 81.9213) (end 148.7424 81.9404) (width 0.254) (layer "F.Cu") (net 4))
 (segment (start 146.1516 81.9213) (end 148.7233 81.9213) (width 0.254) (layer "F.Cu") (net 4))
 (segment (start 148.7424 81.9404) (end 149.225 81.4578) (width 0.254) (layer "F.Cu") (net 4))
 (segment (start 149.225 81.4578) (end 149.225 79.8068) (width 0.254) (layer "F.Cu") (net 4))
 (segment (start 148.7187 82.4213) (end 148.7424 82.3976) (width 0.254) (layer "F.Cu") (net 3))
 (segment (start 146.1516 82.4213) (end 147.5232 82.4213) (width 0.254) (layer "F.Cu") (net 3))
 (segment (start 148.7424 82.3976) (end 149.225 82.8802) (width 0.254) (layer "F.Cu") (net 3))
 (segment (start 147.0232 82.9213) (end 147.5232 82.4213) (width 0.254) (layer "F.Cu") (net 3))
 (segment (start 146.1516 82.9213) (end 147.0232 82.9213) (width 0.254) (layer "F.Cu") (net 3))
 (segment (start 147.5232 82.4213) (end 148.7187 82.4213) (width 0.254) (layer "F.Cu") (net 3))
 (segment (start 149.225 82.8802) (end 149.225 84.4868) (width 0.254) (layer "F.Cu") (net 3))
 (segment (start 138.9126 82.9713) (end 138.9626 82.9213) (width 0.254) (layer "F.Cu") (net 5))
 (segment (start 138.9626 82.9213) (end 141.7516 82.9213) (width 0.254) (layer "F.Cu") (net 5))
 (segment (start 142.2292 84.7709) (end 143.49549 84.7709) (width 0.254) (layer "F.Cu") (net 9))
 (segment (start 144.5237 82.8017) (end 143.5608 81.8388) (width 0.254) (layer "F.Cu") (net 9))
 (segment (start 144.5237 83.74269) (end 144.5237 82.8017) (width 0.254) (layer "F.Cu") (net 9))
 (segment (start 143.49549 84.7709) (end 144.5237 83.74269) (width 0.254) (layer "F.Cu") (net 9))
 (segment (start 141.7516 81.9213) (end 143.4783 81.9213) (width 0.254) (layer "F.Cu") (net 9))
 (segment (start 143.5608 81.915) (end 143.5545 81.9213) (width 0.254) (layer "F.Cu") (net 9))
 (segment (start 143.4783 81.9213) (end 143.5608 81.8388) (width 0.254) (layer "F.Cu") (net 9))
 (segment (start 141.4272 85.5729) (end 142.2292 84.7709) (width 0.254) (layer "F.Cu") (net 9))
 (via (at 143.5608 81.8388) (size 0.8) (drill 0.4) (layers "F.Cu" "B.Cu") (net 9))
 (segment (start 142.6972 86.0809) (end 142.6972 85.1157) (width 0.254) (layer "B.Cu") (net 9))
 (segment (start 142.6972 83.1596) (end 142.6972 82.7024) (width 0.254) (layer "B.Cu") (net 9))
 (segment (start 142.6972 85.7596) (end 142.6972 88.3596) (width 0.254) (layer "B.Cu") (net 9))
 (segment (start 142.6972 82.7024) (end 143.5608 81.8388) (width 0.254) (layer "B.Cu") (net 9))
 (segment (start 142.6972 83.1596) (end 142.6972 85.7596) (width 0.254) (layer "B.Cu") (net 9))
 (segment (start 144.1193 87.1223) (end 144.1196 87.122) (width 0.254) (layer "F.Cu") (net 6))
 (segment (start 143.2791 82.642) (end 143.259666 82.642) (width 0.254) (layer "F.Cu") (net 6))
 (segment (start 143.038966 82.4213) (end 141.7516 82.4213) (width 0.254) (layer "F.Cu") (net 6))
 (segment (start 143.259666 82.642) (end 143.038966 82.4213) (width 0.254) (layer "F.Cu") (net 6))
 (segment (start 143.0782 87.1223) (end 144.1193 87.1223) (width 0.254) (layer "F.Cu") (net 6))
 (segment (start 143.7967 83.1596) (end 143.2791 82.642) (width 0.254) (layer "F.Cu") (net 6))
 (via (at 144.1196 87.122) (size 0.8) (drill 0.4) (layers "F.Cu" "B.Cu") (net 6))
 (via (at 143.7967 83.1596) (size 0.8) (drill 0.4) (layers "F.Cu" "B.Cu") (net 6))
 (segment (start 144.1196 86.514396) (end 144.874396 85.7596) (width 0.254) (layer "B.Cu") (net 6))
 (segment (start 144.874396 83.1596) (end 144.874396 85.7596) (width 0.254) (layer "B.Cu") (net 6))
 (segment (start 144.874396 88.3596) (end 144.874396 85.7596) (width 0.254) (layer "B.Cu") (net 6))
 (segment (start 144.1196 87.122) (end 144.1196 86.514396) (width 0.254) (layer "B.Cu") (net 6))
 (segment (start 143.7967 83.1596) (end 144.874396 83.1596) (width 0.254) (layer "B.Cu") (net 6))
 (segment (start 144.874396 88.6809) (end 144.874396 86.0809) (width 0.254) (layer "B.Cu") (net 6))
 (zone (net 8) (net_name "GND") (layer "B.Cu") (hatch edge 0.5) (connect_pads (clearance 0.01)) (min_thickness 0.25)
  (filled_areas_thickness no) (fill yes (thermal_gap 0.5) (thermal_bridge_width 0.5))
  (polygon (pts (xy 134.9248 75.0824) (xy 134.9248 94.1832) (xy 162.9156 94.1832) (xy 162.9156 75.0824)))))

